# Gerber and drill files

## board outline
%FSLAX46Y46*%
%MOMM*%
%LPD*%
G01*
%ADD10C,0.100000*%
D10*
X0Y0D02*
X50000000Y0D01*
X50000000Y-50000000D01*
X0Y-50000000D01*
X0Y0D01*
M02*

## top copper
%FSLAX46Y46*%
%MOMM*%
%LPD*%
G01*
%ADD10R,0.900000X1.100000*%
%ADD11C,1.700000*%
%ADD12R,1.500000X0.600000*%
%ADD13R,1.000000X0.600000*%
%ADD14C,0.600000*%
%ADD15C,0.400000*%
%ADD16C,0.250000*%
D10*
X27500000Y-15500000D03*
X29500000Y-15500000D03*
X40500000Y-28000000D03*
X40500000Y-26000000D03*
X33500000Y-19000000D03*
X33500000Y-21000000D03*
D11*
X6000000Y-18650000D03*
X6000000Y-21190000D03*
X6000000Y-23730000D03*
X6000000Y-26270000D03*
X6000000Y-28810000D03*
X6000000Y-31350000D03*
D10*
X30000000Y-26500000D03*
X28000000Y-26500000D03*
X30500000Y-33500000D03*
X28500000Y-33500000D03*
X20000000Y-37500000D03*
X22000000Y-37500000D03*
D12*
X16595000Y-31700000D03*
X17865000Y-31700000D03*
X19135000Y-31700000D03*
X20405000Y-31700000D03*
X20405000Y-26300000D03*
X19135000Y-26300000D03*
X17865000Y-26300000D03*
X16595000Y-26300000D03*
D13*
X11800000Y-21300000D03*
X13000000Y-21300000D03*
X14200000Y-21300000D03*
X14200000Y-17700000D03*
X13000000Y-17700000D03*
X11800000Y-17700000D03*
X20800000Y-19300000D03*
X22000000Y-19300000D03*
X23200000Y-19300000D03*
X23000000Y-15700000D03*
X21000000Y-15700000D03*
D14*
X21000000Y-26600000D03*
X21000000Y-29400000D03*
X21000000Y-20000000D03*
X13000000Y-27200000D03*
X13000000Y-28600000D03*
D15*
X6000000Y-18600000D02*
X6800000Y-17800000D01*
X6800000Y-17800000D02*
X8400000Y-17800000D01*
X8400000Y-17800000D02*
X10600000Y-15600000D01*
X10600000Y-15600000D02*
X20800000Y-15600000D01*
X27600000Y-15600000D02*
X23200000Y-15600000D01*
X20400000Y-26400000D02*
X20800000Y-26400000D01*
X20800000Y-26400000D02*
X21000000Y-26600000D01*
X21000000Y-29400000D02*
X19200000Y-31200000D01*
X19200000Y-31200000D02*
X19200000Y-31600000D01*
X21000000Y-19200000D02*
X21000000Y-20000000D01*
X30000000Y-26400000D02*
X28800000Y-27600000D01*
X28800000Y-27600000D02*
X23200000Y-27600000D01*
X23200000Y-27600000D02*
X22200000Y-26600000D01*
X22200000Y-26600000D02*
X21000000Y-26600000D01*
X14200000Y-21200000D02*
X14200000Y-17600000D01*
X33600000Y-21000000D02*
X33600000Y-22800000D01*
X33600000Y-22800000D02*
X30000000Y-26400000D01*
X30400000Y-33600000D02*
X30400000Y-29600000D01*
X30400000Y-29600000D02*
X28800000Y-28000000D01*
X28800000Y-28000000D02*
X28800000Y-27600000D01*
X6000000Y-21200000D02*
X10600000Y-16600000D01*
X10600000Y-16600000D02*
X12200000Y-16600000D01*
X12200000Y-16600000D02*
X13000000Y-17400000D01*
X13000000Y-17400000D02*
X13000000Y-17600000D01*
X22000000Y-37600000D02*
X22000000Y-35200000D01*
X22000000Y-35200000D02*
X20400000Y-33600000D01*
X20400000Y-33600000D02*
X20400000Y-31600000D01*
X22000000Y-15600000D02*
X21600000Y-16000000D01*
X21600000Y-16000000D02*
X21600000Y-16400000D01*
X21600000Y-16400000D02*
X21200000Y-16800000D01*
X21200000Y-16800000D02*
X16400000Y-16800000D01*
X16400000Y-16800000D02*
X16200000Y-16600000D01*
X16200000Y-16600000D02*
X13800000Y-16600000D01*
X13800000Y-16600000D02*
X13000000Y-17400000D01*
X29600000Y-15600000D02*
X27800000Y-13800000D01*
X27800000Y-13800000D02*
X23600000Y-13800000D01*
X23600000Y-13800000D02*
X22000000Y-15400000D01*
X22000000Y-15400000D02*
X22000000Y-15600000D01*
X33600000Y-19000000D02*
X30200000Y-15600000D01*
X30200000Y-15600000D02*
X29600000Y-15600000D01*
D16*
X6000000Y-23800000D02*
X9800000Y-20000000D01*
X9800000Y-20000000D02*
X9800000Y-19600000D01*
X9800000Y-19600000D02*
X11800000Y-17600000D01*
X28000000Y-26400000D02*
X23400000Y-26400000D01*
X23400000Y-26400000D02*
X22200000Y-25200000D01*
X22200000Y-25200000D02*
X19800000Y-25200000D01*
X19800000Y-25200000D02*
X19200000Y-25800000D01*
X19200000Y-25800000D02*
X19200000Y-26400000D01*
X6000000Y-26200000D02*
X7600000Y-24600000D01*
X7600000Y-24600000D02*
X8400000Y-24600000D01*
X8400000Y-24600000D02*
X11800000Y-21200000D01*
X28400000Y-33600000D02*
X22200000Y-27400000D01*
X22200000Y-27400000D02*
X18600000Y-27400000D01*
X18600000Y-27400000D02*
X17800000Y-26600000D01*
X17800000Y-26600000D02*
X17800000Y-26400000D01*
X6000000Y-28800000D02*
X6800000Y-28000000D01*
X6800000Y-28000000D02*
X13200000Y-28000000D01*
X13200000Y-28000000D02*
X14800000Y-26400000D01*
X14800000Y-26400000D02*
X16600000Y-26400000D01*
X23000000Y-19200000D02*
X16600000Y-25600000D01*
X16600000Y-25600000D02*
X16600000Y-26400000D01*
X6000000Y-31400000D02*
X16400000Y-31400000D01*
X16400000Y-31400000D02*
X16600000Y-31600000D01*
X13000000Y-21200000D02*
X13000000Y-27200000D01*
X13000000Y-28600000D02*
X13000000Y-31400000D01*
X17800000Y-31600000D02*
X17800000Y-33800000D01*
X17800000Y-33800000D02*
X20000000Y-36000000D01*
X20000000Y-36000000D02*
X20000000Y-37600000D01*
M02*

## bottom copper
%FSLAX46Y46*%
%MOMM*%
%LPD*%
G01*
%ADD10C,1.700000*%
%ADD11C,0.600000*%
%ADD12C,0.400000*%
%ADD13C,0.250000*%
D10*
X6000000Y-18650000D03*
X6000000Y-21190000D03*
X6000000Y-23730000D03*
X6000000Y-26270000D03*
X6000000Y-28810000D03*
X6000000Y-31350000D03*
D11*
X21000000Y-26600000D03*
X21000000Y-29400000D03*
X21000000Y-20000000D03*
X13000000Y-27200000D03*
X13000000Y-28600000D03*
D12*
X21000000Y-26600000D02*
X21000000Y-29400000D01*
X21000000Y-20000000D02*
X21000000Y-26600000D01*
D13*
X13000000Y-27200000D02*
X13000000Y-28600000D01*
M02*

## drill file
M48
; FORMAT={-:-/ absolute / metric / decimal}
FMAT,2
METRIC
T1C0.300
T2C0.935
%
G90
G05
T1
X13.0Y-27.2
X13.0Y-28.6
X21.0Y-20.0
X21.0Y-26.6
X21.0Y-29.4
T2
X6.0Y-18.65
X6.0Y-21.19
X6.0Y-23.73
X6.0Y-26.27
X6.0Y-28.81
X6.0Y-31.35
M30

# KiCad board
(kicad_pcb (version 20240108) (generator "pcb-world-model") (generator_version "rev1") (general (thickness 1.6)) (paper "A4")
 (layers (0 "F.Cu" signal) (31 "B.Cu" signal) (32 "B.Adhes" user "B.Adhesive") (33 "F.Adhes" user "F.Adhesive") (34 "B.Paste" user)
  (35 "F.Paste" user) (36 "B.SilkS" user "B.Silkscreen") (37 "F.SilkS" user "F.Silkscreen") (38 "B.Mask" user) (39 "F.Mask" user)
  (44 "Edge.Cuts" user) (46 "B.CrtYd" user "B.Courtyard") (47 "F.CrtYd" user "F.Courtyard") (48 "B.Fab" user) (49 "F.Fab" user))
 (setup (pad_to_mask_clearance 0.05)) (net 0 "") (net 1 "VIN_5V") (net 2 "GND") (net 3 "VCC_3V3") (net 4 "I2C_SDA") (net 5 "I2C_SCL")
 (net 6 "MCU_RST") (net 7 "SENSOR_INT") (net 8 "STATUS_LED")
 (gr_rect (start 0.0 0.0) (end 50.0000 50.0000) (stroke (width 0.1) (type default)) (fill none) (layer "Edge.Cuts"))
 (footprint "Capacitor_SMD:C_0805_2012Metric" (layer "F.Cu") (at 28.5000 15.5000 0)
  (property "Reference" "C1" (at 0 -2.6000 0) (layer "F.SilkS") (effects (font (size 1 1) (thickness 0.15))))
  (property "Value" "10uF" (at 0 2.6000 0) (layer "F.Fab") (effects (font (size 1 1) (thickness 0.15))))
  (pad "1" smd rect (at -1.0000 0.0000) (size 0.9000 1.1000) (layers "F.Cu" "F.Paste" "F.Mask") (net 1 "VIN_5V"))
  (pad "2" smd rect (at 1.0000 0.0000) (size 0.9000 1.1000) (layers "F.Cu" "F.Paste" "F.Mask") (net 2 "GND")))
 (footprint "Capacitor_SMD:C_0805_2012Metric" (layer "F.Cu") (at 40.5000 27.0000 90)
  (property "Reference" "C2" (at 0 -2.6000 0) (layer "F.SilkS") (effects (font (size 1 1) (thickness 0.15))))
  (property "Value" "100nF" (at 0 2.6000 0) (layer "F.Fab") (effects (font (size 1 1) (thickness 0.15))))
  (pad "1" smd rect (at -1.0000 0.0000) (size 0.9000 1.1000) (layers "F.Cu" "F.Paste" "F.Mask") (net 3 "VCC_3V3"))
  (pad "2" smd rect (at 1.0000 0.0000) (size 0.9000 1.1000) (layers "F.Cu" "F.Paste" "F.Mask") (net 2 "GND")))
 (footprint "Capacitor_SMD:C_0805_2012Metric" (layer "F.Cu") (at 33.5000 20.0000 270)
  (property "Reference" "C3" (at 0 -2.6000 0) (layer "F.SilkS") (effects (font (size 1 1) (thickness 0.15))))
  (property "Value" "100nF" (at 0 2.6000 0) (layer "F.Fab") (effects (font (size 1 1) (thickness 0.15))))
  (pad "1" smd rect (at -1.0000 0.0000) (size 0.9000 1.1000) (layers "F.Cu" "F.Paste" "F.Mask") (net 3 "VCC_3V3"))
  (pad "2" smd rect (at 1.0000 0.0000) (size 0.9000 1.1000) (layers "F.Cu" "F.Paste" "F.Mask") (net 2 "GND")))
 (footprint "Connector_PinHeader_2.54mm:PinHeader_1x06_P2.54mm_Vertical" (layer "F.Cu") (at 6.0000 25.0000 0) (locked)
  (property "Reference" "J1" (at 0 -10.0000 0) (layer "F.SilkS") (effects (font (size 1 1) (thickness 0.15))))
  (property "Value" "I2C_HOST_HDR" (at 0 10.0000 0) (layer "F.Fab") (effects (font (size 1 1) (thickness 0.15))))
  (pad "1" thru_hole circle (at 0.0000 -6.3500) (size 1.7000 1.7000) (drill 0.9350) (layers "*.Cu" "*.Mask") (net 1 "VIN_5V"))
  (pad "2" thru_hole circle (at 0.0000 -3.8100) (size 1.7000 1.7000) (drill 0.9350) (layers "*.Cu" "*.Mask") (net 2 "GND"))
  (pad "3" thru_hole circle (at 0.0000 -1.2700) (size 1.7000 1.7000) (drill 0.9350) (layers "*.Cu" "*.Mask") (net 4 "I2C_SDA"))
  (pad "4" thru_hole circle (at 0.0000 1.2700) (size 1.7000 1.7000) (drill 0.9350) (layers "*.Cu" "*.Mask") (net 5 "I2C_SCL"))
  (pad "5" thru_hole circle (at 0.0000 3.8100) (size 1.7000 1.7000) (drill 0.9350) (layers "*.Cu" "*.Mask") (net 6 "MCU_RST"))
  (pad "6" thru_hole circle (at 0.0000 6.3500) (size 1.7000 1.7000) (drill 0.9350) (layers "*.Cu" "*.Mask") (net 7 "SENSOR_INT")))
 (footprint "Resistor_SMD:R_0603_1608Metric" (layer "F.Cu") (at 29.0000 26.5000 180)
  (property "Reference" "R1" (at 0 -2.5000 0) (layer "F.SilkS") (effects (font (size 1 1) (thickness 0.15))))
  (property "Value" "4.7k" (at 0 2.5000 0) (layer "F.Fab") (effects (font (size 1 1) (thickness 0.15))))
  (pad "1" smd rect (at -1.0000 0.0000) (size 0.9000 1.1000) (layers "F.Cu" "F.Paste" "F.Mask") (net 3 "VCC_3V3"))
  (pad "2" smd rect (at 1.0000 0.0000) (size 0.9000 1.1000) (layers "F.Cu" "F.Paste" "F.Mask") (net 4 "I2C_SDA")))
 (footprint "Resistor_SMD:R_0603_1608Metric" (layer "F.Cu") (at 29.5000 33.5000 180)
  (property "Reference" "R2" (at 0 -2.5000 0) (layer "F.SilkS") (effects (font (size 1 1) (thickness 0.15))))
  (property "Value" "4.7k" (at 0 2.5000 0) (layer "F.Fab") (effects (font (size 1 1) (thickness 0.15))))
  (pad "1" smd rect (at -1.0000 0.0000) (size 0.9000 1.1000) (layers "F.Cu" "F.Paste" "F.Mask") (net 3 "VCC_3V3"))
  (pad "2" smd rect (at 1.0000 0.0000) (size 0.9000 1.1000) (layers "F.Cu" "F.Paste" "F.Mask") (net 5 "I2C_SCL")))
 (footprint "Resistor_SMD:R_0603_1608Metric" (layer "F.Cu") (at 21.0000 37.5000 0)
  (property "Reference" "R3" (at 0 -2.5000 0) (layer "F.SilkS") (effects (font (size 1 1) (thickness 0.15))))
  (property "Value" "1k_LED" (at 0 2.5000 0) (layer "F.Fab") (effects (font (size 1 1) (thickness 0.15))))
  (pad "1" smd rect (at -1.0000 0.0000) (size 0.9000 1.1000) (layers "F.Cu" "F.Paste" "F.Mask") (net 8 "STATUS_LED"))
  (pad "2" smd rect (at 1.0000 0.0000) (size 0.9000 1.1000) (layers "F.Cu" "F.Paste" "F.Mask") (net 2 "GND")))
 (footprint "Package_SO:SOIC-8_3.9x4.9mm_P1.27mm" (layer "F.Cu") (at 18.5000 29.0000 90)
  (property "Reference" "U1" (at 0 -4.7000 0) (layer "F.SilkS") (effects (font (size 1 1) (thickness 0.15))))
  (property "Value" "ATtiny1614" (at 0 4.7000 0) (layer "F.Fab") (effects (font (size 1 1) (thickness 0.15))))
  (pad "1" smd rect (at -2.7000 -1.9050) (size 1.5000 0.6000) (layers "F.Cu" "F.Paste" "F.Mask") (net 3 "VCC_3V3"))
  (pad "2" smd rect (at -2.7000 -0.6350) (size 1.5000 0.6000) (layers "F.Cu" "F.Paste" "F.Mask") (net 4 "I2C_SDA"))
  (pad "3" smd rect (at -2.7000 0.6350) (size 1.5000 0.6000) (layers "F.Cu" "F.Paste" "F.Mask") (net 5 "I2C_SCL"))
  (pad "4" smd rect (at -2.7000 1.9050) (size 1.5000 0.6000) (layers "F.Cu" "F.Paste" "F.Mask") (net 6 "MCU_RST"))
  (pad "5" smd rect (at 2.7000 1.9050) (size 1.5000 0.6000) (layers "F.Cu" "F.Paste" "F.Mask") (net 7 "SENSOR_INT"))
  (pad "6" smd rect (at 2.7000 0.6350) (size 1.5000 0.6000) (layers "F.Cu" "F.Paste" "F.Mask") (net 8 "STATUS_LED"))
  (pad "7" smd rect (at 2.7000 -0.6350) (size 1.5000 0.6000) (layers "F.Cu" "F.Paste" "F.Mask") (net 3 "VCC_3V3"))
  (pad "8" smd rect (at 2.7000 -1.9050) (size 1.5000 0.6000) (layers "F.Cu" "F.Paste" "F.Mask") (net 2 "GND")))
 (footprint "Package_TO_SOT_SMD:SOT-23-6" (layer "F.Cu") (at 13.0000 19.5000 90)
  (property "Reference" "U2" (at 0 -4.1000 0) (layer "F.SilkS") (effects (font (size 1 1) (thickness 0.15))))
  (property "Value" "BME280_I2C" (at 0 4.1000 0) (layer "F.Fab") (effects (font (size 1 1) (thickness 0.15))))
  (pad "1" smd rect (at -1.8000 -1.2000) (size 1.0000 0.6000) (layers "F.Cu" "F.Paste" "F.Mask") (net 3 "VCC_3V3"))
  (pad "2" smd rect (at -1.8000 0.0000) (size 1.0000 0.6000) (layers "F.Cu" "F.Paste" "F.Mask") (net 2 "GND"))
  (pad "3" smd rect (at -1.8000 1.2000) (size 1.0000 0.6000) (layers "F.Cu" "F.Paste" "F.Mask") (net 4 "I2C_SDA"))
  (pad "4" smd rect (at 1.8000 1.2000) (size 1.0000 0.6000) (layers "F.Cu" "F.Paste" "F.Mask") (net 5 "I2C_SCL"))
  (pad "5" smd rect (at 1.8000 0.0000) (size 1.0000 0.6000) (layers "F.Cu" "F.Paste" "F.Mask") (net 7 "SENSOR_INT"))
  (pad "6" smd rect (at 1.8000 -1.2000) (size 1.0000 0.6000) (layers "F.Cu" "F.Paste" "F.Mask") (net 3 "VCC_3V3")))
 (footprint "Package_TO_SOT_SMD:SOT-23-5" (layer "F.Cu") (at 22.0000 17.5000 90)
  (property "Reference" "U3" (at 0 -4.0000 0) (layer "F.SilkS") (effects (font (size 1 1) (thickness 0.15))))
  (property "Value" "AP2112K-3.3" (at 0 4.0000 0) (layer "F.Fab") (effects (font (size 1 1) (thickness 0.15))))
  (pad "1" smd rect (at -1.8000 -1.2000) (size 1.0000 0.6000) (layers "F.Cu" "F.Paste" "F.Mask") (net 1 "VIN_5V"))
  (pad "2" smd rect (at -1.8000 0.0000) (size 1.0000 0.6000) (layers "F.Cu" "F.Paste" "F.Mask") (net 2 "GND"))
  (pad "3" smd rect (at -1.8000 1.2000) (size 1.0000 0.6000) (layers "F.Cu" "F.Paste" "F.Mask") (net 1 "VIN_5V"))
  (pad "4" smd rect (at 1.8000 1.0000) (size 1.0000 0.6000) (layers "F.Cu" "F.Paste" "F.Mask") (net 3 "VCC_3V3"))
  (pad "5" smd rect (at 1.8000 -1.0000) (size 1.0000 0.6000) (layers "F.Cu" "F.Paste" "F.Mask") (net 6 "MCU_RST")))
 (segment (start 6.0000 18.6000) (end 6.8000 17.8000) (width 0.4000) (layer "F.Cu") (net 1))
 (segment (start 6.8000 17.8000) (end 8.4000 17.8000) (width 0.4000) (layer "F.Cu") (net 1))
 (segment (start 8.4000 17.8000) (end 10.6000 15.6000) (width 0.4000) (layer "F.Cu") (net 1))
 (segment (start 10.6000 15.6000) (end 20.8000 15.6000) (width 0.4000) (layer "F.Cu") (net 1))
 (segment (start 27.6000 15.6000) (end 23.2000 15.6000) (width 0.4000) (layer "F.Cu") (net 1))
 (segment (start 20.4000 26.4000) (end 20.8000 26.4000) (width 0.4000) (layer "F.Cu") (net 3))
 (segment (start 20.8000 26.4000) (end 21.0000 26.6000) (width 0.4000) (layer "F.Cu") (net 3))
 (segment (start 21.0000 26.6000) (end 21.0000 29.4000) (width 0.4000) (layer "B.Cu") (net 3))
 (segment (start 21.0000 29.4000) (end 19.2000 31.2000) (width 0.4000) (layer "F.Cu") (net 3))
 (segment (start 19.2000 31.2000) (end 19.2000 31.6000) (width 0.4000) (layer "F.Cu") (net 3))
 (segment (start 21.0000 19.2000) (end 21.0000 20.0000) (width 0.4000) (layer "F.Cu") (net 3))
 (segment (start 21.0000 20.0000) (end 21.0000 26.6000) (width 0.4000) (layer "B.Cu") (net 3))
 (segment (start 30.0000 26.4000) (end 28.8000 27.6000) (width 0.4000) (layer "F.Cu") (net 3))
 (segment (start 28.8000 27.6000) (end 23.2000 27.6000) (width 0.4000) (layer "F.Cu") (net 3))
 (segment (start 23.2000 27.6000) (end 22.2000 26.6000) (width 0.4000) (layer "F.Cu") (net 3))
 (segment (start 22.2000 26.6000) (end 21.0000 26.6000) (width 0.4000) (layer "F.Cu") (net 3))
 (segment (start 14.2000 21.2000) (end 14.2000 17.6000) (width 0.4000) (layer "F.Cu") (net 3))
 (segment (start 33.6000 21.0000) (end 33.6000 22.8000) (width 0.4000) (layer "F.Cu") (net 3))
 (segment (start 33.6000 22.8000) (end 30.0000 26.4000) (width 0.4000) (layer "F.Cu") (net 3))
 (segment (start 30.4000 33.6000) (end 30.4000 29.6000) (width 0.4000) (layer "F.Cu") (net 3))
 (segment (start 30.4000 29.6000) (end 28.8000 28.0000) (width 0.4000) (layer "F.Cu") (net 3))
 (segment (start 28.8000 28.0000) (end 28.8000 27.6000) (width 0.4000) (layer "F.Cu") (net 3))
 (segment (start 6.0000 21.2000) (end 10.6000 16.6000) (width 0.4000) (layer "F.Cu") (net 2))
 (segment (start 10.6000 16.6000) (end 12.2000 16.6000) (width 0.4000) (layer "F.Cu") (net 2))
 (segment (start 12.2000 16.6000) (end 13.0000 17.4000) (width 0.4000) (layer "F.Cu") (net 2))
 (segment (start 13.0000 17.4000) (end 13.0000 17.6000) (width 0.4000) (layer "F.Cu") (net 2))
 (segment (start 22.0000 37.6000) (end 22.0000 35.2000) (width 0.4000) (layer "F.Cu") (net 2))
 (segment (start 22.0000 35.2000) (end 20.4000 33.6000) (width 0.4000) (layer "F.Cu") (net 2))
 (segment (start 20.4000 33.6000) (end 20.4000 31.6000) (width 0.4000) (layer "F.Cu") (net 2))
 (segment (start 22.0000 15.6000) (end 21.6000 16.0000) (width 0.4000) (layer "F.Cu") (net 2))
 (segment (start 21.6000 16.0000) (end 21.6000 16.4000) (width 0.4000) (layer "F.Cu") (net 2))
 (segment (start 21.6000 16.4000) (end 21.2000 16.8000) (width 0.4000) (layer "F.Cu") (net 2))
 (segment (start 21.2000 16.8000) (end 16.4000 16.8000) (width 0.4000) (layer "F.Cu") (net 2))
 (segment (start 16.4000 16.8000) (end 16.2000 16.6000) (width 0.4000) (layer "F.Cu") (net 2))
 (segment (start 16.2000 16.6000) (end 13.8000 16.6000) (width 0.4000) (layer "F.Cu") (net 2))
 (segment (start 13.8000 16.6000) (end 13.0000 17.4000) (width 0.4000) (layer "F.Cu") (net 2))
 (segment (start 29.6000 15.6000) (end 27.8000 13.8000) (width 0.4000) (layer "F.Cu") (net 2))
 (segment (start 27.8000 13.8000) (end 23.6000 13.8000) (width 0.4000) (layer "F.Cu") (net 2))
 (segment (start 23.6000 13.8000) (end 22.0000 15.4000) (width 0.4000) (layer "F.Cu") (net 2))
 (segment (start 22.0000 15.4000) (end 22.0000 15.6000) (width 0.4000) (layer "F.Cu") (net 2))
 (segment (start 33.6000 19.0000) (end 30.2000 15.6000) (width 0.4000) (layer "F.Cu") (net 2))
 (segment (start 30.2000 15.6000) (end 29.6000 15.6000) (width 0.4000) (layer "F.Cu") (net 2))
 (segment (start 6.0000 23.8000) (end 9.8000 20.0000) (width 0.2500) (layer "F.Cu") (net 4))
 (segment (start 9.8000 20.0000) (end 9.8000 19.6000) (width 0.2500) (layer "F.Cu") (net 4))
 (segment (start 9.8000 19.6000) (end 11.8000 17.6000) (width 0.2500) (layer "F.Cu") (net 4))
 (segment (start 28.0000 26.4000) (end 23.4000 26.4000) (width 0.2500) (layer "F.Cu") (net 4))
 (segment (start 23.4000 26.4000) (end 22.2000 25.2000) (width 0.2500) (layer "F.Cu") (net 4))
 (segment (start 22.2000 25.2000) (end 19.8000 25.2000) (width 0.2500) (layer "F.Cu") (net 4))
 (segment (start 19.8000 25.2000) (end 19.2000 25.8000) (width 0.2500) (layer "F.Cu") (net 4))
 (segment (start 19.2000 25.8000) (end 19.2000 26.4000) (width 0.2500) (layer "F.Cu") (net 4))
 (segment (start 6.0000 26.2000) (end 7.6000 24.6000) (width 0.2500) (layer "F.Cu") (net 5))
 (segment (start 7.6000 24.6000) (end 8.4000 24.6000) (width 0.2500) (layer "F.Cu") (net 5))
 (segment (start 8.4000 24.6000) (end 11.8000 21.2000) (width 0.2500) (layer "F.Cu") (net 5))
 (segment (start 28.4000 33.6000) (end 22.2000 27.4000) (width 0.2500) (layer "F.Cu") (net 5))
 (segment (start 22.2000 27.4000) (end 18.6000 27.4000) (width 0.2500) (layer "F.Cu") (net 5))
 (segment (start 18.6000 27.4000) (end 17.8000 26.6000) (width 0.2500) (layer "F.Cu") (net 5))
 (segment (start 17.8000 26.6000) (end 17.8000 26.4000) (width 0.2500) (layer "F.Cu") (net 5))
 (segment (start 6.0000 28.8000) (end 6.8000 28.0000) (width 0.2500) (layer "F.Cu") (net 6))
 (segment (start 6.8000 28.0000) (end 13.2000 28.0000) (width 0.2500) (layer "F.Cu") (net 6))
 (segment (start 13.2000 28.0000) (end 14.8000 26.4000) (width 0.2500) (layer "F.Cu") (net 6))
 (segment (start 14.8000 26.4000) (end 16.6000 26.4000) (width 0.2500) (layer "F.Cu") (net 6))
 (segment (start 23.0000 19.2000) (end 16.6000 25.6000) (width 0.2500) (layer "F.Cu") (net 6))
 (segment (start 16.6000 25.6000) (end 16.6000 26.4000) (width 0.2500) (layer "F.Cu") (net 6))
 (segment (start 6.0000 31.4000) (end 16.4000 31.4000) (width 0.2500) (layer "F.Cu") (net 7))
 (segment (start 16.4000 31.4000) (end 16.6000 31.6000) (width 0.2500) (layer "F.Cu") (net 7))
 (segment (start 13.0000 21.2000) (end 13.0000 27.2000) (width 0.2500) (layer "F.Cu") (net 7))
 (segment (start 13.0000 27.2000) (end 13.0000 28.6000) (width 0.2500) (layer "B.Cu") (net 7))
 (segment (start 13.0000 28.6000) (end 13.0000 31.4000) (width 0.2500) (layer "F.Cu") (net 7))
 (segment (start 17.8000 31.6000) (end 17.8000 33.8000) (width 0.2500) (layer "F.Cu") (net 8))
 (segment (start 17.8000 33.8000) (end 20.0000 36.0000) (width 0.2500) (layer "F.Cu") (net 8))
 (segment (start 20.0000 36.0000) (end 20.0000 37.6000) (width 0.2500) (layer "F.Cu") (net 8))
 (via (at 21.0000 26.6000) (size 0.6000) (drill 0.3000) (layers "F.Cu" "B.Cu") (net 3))
 (via (at 21.0000 29.4000) (size 0.6000) (drill 0.3000) (layers "F.Cu" "B.Cu") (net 3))
 (via (at 21.0000 20.0000) (size 0.6000) (drill 0.3000) (layers "F.Cu" "B.Cu") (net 3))
 (via (at 13.0000 27.2000) (size 0.6000) (drill 0.3000) (layers "F.Cu" "B.Cu") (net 7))
 (via (at 13.0000 28.6000) (size 0.6000) (drill 0.3000) (layers "F.Cu" "B.Cu") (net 7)))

